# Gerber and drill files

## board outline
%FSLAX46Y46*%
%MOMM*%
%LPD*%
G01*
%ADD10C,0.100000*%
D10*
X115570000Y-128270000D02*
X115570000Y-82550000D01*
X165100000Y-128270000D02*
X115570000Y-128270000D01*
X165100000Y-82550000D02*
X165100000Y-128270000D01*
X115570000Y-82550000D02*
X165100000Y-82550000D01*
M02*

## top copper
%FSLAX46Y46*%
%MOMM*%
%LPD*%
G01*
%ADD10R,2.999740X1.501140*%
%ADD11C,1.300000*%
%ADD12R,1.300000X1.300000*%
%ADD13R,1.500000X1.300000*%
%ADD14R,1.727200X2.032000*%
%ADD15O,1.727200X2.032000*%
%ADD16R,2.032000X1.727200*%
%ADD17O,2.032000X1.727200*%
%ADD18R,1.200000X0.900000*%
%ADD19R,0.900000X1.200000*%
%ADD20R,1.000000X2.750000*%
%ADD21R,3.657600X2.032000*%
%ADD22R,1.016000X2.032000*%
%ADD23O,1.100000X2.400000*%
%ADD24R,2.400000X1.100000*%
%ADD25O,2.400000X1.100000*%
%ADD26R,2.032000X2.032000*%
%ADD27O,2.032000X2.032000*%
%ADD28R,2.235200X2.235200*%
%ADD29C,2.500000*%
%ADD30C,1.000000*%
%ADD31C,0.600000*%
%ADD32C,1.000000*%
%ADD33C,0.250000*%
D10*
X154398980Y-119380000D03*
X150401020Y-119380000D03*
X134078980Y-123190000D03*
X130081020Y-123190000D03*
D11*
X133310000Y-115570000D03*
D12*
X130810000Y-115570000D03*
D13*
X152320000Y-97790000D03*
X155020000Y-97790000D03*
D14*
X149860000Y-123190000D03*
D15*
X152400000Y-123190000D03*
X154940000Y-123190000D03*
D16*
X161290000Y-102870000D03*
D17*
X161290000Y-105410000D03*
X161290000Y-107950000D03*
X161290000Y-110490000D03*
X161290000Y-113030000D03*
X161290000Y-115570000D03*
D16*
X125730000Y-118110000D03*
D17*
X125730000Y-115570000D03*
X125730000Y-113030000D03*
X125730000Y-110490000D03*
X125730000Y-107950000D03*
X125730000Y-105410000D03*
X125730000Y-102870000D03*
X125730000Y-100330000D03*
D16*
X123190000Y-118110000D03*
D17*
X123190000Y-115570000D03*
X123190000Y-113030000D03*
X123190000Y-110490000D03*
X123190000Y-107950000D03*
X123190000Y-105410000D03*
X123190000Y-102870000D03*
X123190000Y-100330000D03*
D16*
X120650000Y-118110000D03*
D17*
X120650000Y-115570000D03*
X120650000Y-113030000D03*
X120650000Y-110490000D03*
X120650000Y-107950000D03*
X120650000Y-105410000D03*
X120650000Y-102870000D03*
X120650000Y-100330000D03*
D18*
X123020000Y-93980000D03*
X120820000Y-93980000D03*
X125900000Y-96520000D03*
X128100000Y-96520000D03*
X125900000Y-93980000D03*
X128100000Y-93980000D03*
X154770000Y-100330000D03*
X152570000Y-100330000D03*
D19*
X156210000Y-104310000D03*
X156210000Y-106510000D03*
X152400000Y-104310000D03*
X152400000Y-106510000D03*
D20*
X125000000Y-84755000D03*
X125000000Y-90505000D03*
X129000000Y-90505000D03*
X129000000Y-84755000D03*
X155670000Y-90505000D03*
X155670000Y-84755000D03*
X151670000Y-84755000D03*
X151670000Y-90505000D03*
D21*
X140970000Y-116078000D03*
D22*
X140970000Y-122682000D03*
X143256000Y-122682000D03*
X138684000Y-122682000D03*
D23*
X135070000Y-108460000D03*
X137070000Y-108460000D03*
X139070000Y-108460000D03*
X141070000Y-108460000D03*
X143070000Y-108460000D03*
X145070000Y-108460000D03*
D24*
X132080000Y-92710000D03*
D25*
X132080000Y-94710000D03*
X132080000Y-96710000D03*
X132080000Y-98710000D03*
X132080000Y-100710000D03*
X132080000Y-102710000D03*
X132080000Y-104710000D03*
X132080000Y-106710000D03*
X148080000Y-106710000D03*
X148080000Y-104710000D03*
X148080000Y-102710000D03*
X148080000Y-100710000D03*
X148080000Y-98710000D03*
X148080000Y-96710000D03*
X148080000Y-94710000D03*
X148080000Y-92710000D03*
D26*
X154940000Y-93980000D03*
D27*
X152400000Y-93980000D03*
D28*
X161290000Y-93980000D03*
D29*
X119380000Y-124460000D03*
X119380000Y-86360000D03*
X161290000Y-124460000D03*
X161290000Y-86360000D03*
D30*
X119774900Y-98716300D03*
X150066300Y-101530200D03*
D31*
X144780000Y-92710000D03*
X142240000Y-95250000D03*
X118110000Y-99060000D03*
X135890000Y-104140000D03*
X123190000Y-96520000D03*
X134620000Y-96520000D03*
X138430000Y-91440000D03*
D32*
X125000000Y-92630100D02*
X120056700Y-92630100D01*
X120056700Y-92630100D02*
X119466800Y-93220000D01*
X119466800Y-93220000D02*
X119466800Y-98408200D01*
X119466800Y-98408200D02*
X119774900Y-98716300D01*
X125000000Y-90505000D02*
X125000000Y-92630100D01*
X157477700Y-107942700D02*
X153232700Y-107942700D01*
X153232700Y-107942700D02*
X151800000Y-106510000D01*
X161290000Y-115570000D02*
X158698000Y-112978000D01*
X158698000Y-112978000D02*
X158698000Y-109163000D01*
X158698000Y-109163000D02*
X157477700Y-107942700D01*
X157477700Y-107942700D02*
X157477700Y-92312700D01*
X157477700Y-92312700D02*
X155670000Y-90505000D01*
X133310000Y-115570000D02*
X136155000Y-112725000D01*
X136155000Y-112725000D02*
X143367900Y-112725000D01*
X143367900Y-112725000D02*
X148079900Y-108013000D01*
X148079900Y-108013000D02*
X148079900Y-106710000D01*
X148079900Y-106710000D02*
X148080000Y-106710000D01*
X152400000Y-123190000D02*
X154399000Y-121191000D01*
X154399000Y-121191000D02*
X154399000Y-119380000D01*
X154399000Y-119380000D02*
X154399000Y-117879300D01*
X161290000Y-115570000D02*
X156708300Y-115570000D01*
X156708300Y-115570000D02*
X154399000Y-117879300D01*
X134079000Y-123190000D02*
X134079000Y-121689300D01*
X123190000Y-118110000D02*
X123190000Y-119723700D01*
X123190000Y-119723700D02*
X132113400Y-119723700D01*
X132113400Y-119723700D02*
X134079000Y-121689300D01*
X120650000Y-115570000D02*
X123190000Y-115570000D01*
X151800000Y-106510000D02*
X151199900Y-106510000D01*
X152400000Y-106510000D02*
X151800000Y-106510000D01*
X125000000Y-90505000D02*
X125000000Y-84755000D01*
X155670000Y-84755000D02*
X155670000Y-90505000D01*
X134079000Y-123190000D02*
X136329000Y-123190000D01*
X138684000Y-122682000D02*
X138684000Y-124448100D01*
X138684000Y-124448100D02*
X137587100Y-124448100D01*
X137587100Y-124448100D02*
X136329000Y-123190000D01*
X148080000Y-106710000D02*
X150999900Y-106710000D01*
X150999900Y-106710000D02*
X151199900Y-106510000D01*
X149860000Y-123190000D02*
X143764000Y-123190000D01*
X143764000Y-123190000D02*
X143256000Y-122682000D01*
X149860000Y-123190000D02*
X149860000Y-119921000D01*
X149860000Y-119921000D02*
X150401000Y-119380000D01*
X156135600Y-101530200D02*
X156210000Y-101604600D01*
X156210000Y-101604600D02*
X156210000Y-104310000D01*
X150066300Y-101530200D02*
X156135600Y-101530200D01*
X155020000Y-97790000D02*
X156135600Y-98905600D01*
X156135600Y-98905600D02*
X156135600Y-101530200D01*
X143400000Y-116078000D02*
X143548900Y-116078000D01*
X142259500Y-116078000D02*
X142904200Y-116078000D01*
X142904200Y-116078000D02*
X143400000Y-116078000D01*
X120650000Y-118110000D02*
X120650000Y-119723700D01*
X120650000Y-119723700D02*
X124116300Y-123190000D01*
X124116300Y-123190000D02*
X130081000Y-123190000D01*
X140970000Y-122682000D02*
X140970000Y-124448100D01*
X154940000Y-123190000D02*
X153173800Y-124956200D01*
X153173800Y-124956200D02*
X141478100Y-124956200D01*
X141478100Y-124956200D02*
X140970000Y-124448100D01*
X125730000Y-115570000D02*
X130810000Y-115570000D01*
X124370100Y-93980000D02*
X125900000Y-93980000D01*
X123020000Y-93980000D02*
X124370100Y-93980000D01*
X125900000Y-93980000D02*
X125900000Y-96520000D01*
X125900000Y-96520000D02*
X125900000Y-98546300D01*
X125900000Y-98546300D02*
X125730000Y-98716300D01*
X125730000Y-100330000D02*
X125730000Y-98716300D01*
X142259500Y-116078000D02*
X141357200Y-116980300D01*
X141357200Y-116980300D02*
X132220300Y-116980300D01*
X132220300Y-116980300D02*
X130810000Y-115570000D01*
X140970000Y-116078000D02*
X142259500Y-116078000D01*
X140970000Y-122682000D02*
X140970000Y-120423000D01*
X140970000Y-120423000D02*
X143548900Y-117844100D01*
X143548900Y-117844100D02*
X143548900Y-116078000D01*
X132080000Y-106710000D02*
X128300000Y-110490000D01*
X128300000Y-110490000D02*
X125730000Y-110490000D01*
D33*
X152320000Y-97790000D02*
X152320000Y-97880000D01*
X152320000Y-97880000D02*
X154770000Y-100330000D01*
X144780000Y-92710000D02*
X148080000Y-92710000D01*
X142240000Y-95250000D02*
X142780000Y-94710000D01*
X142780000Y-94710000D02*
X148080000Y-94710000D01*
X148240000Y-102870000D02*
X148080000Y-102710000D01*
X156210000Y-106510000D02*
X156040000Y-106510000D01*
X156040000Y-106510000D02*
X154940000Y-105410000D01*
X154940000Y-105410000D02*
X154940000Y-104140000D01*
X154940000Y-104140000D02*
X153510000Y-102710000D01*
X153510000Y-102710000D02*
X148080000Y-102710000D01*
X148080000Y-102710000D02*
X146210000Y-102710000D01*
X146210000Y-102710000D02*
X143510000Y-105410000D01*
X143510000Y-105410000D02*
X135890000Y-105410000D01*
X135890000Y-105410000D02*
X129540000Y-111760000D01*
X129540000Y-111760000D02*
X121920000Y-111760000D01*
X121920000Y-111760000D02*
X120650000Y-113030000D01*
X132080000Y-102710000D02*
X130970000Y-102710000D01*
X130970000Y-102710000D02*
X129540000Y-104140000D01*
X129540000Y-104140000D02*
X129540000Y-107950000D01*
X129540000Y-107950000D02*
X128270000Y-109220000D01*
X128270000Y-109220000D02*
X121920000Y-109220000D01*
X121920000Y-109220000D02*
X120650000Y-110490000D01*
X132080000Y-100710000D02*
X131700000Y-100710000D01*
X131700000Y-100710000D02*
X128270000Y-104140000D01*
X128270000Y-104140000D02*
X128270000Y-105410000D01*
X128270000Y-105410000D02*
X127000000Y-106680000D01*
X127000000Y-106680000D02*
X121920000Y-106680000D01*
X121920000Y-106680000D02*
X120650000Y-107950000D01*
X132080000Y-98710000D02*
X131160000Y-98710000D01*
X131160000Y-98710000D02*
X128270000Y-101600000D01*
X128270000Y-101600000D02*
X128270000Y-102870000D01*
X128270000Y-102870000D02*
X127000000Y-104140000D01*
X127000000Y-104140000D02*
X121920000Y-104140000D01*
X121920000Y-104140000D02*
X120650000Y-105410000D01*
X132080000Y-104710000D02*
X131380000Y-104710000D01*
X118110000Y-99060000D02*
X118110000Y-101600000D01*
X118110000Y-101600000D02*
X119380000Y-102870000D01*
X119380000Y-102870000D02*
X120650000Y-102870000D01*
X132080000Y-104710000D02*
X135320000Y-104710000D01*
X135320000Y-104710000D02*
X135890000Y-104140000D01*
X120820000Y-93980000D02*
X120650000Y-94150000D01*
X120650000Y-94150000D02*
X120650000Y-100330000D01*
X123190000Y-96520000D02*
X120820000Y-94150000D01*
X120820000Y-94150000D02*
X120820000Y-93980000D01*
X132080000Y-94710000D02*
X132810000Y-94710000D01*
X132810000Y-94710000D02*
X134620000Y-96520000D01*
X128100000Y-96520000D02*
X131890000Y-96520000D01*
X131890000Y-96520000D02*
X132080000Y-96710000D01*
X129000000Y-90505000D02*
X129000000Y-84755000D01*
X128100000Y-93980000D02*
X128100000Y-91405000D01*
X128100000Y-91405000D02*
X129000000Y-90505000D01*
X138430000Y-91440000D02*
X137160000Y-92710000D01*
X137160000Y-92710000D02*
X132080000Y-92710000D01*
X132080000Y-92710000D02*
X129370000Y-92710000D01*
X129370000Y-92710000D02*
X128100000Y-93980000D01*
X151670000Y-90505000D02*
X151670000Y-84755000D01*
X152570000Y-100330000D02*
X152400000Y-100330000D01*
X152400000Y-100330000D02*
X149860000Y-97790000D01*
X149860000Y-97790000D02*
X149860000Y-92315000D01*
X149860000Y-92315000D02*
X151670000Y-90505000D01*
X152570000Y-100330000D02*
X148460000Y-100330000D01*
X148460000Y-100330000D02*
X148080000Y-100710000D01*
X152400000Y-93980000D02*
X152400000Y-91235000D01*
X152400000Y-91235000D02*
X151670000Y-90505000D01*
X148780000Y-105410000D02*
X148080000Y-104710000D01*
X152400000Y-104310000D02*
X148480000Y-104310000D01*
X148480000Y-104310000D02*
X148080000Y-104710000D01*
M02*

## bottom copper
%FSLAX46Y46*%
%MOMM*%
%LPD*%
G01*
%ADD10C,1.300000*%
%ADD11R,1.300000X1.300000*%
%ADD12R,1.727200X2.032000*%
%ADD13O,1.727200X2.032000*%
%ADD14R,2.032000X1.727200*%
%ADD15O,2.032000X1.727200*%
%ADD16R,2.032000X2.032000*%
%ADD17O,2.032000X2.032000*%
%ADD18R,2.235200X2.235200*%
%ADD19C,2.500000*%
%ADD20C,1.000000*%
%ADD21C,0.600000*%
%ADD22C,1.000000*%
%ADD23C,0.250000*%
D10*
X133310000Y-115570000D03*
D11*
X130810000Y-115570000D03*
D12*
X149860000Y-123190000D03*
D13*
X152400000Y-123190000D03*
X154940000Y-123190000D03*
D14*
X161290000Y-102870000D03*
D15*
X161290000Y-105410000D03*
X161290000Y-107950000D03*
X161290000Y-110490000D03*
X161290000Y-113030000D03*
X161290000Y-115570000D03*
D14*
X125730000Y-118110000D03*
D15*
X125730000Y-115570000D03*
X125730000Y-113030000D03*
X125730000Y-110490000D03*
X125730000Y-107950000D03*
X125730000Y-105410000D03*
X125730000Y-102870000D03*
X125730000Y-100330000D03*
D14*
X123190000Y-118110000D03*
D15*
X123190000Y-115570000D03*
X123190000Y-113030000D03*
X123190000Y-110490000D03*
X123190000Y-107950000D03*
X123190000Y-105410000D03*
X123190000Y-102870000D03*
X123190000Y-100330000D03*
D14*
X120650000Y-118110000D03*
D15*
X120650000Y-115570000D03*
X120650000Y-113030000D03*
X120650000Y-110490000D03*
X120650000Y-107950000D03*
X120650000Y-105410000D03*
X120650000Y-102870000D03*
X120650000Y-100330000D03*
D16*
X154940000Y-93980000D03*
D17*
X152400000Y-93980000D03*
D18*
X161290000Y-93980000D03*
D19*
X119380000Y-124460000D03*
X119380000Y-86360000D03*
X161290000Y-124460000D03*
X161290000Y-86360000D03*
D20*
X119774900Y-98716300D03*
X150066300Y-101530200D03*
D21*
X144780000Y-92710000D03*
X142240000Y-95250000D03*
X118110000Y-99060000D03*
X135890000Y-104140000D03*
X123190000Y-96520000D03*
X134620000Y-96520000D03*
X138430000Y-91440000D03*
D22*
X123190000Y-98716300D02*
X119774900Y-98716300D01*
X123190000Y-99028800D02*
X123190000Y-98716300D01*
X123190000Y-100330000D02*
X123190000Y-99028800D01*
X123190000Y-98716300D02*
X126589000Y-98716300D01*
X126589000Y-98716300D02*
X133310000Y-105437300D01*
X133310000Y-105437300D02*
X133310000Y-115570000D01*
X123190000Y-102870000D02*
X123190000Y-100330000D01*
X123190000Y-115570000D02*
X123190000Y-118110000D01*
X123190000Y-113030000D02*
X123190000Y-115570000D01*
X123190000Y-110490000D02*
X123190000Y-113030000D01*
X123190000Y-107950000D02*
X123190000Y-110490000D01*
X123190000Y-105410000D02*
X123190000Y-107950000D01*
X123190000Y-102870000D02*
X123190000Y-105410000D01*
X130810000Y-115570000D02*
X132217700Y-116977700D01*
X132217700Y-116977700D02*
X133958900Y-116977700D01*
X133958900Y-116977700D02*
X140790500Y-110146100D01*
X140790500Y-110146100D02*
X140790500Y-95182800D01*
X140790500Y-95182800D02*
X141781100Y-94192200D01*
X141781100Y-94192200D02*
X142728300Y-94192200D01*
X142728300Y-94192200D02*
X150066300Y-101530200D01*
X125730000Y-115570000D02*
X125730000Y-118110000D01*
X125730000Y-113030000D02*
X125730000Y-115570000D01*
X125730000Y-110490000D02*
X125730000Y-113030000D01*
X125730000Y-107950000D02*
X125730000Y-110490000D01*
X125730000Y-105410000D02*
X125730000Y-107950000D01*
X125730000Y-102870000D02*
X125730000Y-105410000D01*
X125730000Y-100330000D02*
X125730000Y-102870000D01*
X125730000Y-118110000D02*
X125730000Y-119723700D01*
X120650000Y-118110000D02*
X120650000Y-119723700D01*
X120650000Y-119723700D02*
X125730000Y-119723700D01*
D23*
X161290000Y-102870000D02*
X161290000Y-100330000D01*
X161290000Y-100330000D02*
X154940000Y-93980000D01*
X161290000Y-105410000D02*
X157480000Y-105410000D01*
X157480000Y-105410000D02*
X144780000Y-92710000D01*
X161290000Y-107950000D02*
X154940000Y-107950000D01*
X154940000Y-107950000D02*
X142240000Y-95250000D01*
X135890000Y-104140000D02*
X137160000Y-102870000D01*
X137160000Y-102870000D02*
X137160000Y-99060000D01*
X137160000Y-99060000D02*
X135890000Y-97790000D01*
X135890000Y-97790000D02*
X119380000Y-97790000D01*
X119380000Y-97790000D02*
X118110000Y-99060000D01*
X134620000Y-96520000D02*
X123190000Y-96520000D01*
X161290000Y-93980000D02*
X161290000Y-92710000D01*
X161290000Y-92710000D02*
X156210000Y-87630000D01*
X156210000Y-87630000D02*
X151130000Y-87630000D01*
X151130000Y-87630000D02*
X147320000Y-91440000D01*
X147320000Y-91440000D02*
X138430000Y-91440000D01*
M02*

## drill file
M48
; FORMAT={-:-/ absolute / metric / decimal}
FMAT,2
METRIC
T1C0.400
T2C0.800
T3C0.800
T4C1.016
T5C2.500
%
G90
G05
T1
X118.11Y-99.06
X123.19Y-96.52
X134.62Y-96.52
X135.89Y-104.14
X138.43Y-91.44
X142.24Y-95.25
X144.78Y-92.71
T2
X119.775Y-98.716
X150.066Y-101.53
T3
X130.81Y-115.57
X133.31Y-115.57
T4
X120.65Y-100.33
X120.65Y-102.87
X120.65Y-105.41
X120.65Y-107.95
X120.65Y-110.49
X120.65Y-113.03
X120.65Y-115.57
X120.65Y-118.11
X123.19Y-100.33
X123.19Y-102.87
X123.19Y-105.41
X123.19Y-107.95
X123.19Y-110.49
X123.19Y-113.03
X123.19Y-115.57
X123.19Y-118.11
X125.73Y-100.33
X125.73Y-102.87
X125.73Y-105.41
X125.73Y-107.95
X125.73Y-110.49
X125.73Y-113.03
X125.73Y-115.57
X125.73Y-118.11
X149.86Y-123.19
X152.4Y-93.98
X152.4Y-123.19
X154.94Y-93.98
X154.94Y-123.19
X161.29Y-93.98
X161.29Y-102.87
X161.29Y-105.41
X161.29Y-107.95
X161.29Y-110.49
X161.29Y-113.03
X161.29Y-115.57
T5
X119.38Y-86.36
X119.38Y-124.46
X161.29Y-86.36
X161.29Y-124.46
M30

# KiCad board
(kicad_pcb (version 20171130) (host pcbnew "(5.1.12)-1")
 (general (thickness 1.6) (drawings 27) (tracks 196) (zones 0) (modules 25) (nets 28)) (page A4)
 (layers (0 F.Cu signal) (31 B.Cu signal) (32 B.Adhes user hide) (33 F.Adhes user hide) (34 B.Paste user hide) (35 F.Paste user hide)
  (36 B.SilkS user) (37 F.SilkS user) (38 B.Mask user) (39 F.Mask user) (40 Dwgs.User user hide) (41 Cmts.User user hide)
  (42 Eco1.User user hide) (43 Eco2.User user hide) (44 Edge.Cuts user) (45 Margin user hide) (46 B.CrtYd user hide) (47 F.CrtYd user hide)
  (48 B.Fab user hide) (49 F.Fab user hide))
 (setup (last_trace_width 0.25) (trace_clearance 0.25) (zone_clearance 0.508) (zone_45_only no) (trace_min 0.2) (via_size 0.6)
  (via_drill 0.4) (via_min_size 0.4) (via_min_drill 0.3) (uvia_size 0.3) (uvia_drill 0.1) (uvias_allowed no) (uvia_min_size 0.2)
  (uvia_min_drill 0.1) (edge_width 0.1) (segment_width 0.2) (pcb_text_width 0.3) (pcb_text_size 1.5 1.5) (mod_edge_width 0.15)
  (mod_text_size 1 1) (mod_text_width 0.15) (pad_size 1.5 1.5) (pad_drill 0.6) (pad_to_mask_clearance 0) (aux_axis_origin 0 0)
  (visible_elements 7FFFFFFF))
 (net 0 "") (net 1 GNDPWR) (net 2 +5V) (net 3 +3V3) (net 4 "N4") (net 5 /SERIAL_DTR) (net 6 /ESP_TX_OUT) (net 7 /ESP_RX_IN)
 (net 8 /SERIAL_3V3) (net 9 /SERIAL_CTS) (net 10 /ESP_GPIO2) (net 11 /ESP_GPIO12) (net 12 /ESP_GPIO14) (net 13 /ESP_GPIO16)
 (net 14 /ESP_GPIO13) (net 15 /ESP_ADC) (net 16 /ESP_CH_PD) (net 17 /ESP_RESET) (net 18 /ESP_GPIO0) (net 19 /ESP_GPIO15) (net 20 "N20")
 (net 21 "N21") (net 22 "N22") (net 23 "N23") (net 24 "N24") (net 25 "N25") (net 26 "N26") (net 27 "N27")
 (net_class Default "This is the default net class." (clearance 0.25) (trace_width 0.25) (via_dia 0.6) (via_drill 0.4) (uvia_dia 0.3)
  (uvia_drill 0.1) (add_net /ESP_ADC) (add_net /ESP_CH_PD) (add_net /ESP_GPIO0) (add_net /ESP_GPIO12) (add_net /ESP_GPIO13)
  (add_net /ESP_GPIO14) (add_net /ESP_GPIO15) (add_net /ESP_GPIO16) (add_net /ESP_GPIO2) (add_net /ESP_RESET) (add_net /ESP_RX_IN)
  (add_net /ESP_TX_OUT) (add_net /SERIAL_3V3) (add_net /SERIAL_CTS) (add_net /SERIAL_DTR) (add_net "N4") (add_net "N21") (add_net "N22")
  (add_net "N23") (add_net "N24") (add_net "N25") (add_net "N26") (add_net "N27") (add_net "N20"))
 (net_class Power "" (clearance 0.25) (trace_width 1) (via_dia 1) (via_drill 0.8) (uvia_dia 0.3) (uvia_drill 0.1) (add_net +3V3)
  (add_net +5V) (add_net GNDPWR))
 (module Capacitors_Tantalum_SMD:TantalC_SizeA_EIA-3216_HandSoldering (layer F.Cu) (at 152.4 119.38)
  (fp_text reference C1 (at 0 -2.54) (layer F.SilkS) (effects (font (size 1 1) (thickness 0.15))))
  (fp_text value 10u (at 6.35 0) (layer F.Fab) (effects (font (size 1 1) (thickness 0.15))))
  (pad 2 smd rect (at 1.99898 0) (size 2.99974 1.50114) (layers F.Cu F.Paste F.Mask) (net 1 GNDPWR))
  (pad 1 smd rect (at -1.99898 0) (size 2.99974 1.50114) (layers F.Cu F.Paste F.Mask) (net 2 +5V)))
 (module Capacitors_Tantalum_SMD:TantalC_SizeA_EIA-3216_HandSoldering (layer F.Cu) (at 132.08 123.19)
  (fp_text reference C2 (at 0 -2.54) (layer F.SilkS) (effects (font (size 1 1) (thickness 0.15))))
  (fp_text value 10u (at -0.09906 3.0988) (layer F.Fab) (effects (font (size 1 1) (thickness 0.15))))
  (pad 2 smd rect (at 1.99898 0) (size 2.99974 1.50114) (layers F.Cu F.Paste F.Mask) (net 1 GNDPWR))
  (pad 1 smd rect (at -1.99898 0) (size 2.99974 1.50114) (layers F.Cu F.Paste F.Mask) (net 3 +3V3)))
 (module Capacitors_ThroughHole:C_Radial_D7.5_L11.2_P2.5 (layer F.Cu) (at 130.81 115.57)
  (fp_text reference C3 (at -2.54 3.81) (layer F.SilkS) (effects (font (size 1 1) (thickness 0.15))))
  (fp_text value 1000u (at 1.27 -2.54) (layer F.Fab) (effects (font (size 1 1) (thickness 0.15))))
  (pad 2 thru_hole circle (at 2.5 0) (size 1.3 1.3) (drill 0.8) (layers *.Cu *.Mask F.SilkS) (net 1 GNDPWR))
  (pad 1 thru_hole rect (at 0 0) (size 1.3 1.3) (drill 0.8) (layers *.Cu *.Mask F.SilkS) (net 3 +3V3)))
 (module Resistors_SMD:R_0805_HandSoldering (layer F.Cu) (at 153.67 97.79)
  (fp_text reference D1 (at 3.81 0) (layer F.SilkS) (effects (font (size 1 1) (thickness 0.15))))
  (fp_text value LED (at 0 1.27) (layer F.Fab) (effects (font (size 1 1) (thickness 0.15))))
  (pad 1 smd rect (at -1.35 0) (size 1.5 1.3) (layers F.Cu F.Paste F.Mask) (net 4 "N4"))
  (pad 2 smd rect (at 1.35 0) (size 1.5 1.3) (layers F.Cu F.Paste F.Mask) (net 3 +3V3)))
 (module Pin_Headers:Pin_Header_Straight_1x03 (layer F.Cu) (at 149.86 123.19 90)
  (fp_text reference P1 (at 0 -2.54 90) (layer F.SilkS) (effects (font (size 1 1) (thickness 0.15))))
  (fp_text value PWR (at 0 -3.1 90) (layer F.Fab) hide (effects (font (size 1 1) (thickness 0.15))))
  (pad 1 thru_hole rect (at 0 0 90) (size 2.032 1.7272) (drill 1.016) (layers *.Cu *.Mask F.SilkS) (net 2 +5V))
  (pad 2 thru_hole oval (at 0 2.54 90) (size 2.032 1.7272) (drill 1.016) (layers *.Cu *.Mask F.SilkS) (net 1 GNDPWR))
  (pad 3 thru_hole oval (at 0 5.08 90) (size 2.032 1.7272) (drill 1.016) (layers *.Cu *.Mask F.SilkS) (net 3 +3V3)))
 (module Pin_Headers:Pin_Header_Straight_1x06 (layer F.Cu) (at 161.29 102.87)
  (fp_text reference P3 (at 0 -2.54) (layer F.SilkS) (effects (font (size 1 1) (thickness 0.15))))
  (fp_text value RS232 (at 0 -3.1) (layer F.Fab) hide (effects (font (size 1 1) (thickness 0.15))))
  (pad 1 thru_hole rect (at 0 0) (size 2.032 1.7272) (drill 1.016) (layers *.Cu *.Mask F.SilkS) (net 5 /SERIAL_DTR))
  (pad 2 thru_hole oval (at 0 2.54) (size 2.032 1.7272) (drill 1.016) (layers *.Cu *.Mask F.SilkS) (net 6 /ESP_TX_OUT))
  (pad 3 thru_hole oval (at 0 5.08) (size 2.032 1.7272) (drill 1.016) (layers *.Cu *.Mask F.SilkS) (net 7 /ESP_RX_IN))
  (pad 4 thru_hole oval (at 0 7.62) (size 2.032 1.7272) (drill 1.016) (layers *.Cu *.Mask F.SilkS) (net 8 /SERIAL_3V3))
  (pad 5 thru_hole oval (at 0 10.16) (size 2.032 1.7272) (drill 1.016) (layers *.Cu *.Mask F.SilkS) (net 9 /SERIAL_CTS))
  (pad 6 thru_hole oval (at 0 12.7) (size 2.032 1.7272) (drill 1.016) (layers *.Cu *.Mask F.SilkS) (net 1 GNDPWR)))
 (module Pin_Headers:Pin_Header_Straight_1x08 (layer F.Cu) (at 125.73 118.11 180)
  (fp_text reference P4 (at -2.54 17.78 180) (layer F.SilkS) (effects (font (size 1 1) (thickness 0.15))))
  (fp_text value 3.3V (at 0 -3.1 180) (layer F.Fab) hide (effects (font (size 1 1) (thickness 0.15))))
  (pad 1 thru_hole rect (at 0 0 180) (size 2.032 1.7272) (drill 1.016) (layers *.Cu *.Mask F.SilkS) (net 3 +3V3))
  (pad 2 thru_hole oval (at 0 2.54 180) (size 2.032 1.7272) (drill 1.016) (layers *.Cu *.Mask F.SilkS) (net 3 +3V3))
  (pad 3 thru_hole oval (at 0 5.08 180) (size 2.032 1.7272) (drill 1.016) (layers *.Cu *.Mask F.SilkS) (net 3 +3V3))
  (pad 4 thru_hole oval (at 0 7.62 180) (size 2.032 1.7272) (drill 1.016) (layers *.Cu *.Mask F.SilkS) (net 3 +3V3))
  (pad 5 thru_hole oval (at 0 10.16 180) (size 2.032 1.7272) (drill 1.016) (layers *.Cu *.Mask F.SilkS) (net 3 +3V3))
  (pad 6 thru_hole oval (at 0 12.7 180) (size 2.032 1.7272) (drill 1.016) (layers *.Cu *.Mask F.SilkS) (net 3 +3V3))
  (pad 7 thru_hole oval (at 0 15.24 180) (size 2.032 1.7272) (drill 1.016) (layers *.Cu *.Mask F.SilkS) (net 3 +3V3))
  (pad 8 thru_hole oval (at 0 17.78 180) (size 2.032 1.7272) (drill 1.016) (layers *.Cu *.Mask F.SilkS) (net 3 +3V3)))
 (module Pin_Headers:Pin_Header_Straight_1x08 (layer F.Cu) (at 123.19 118.11 180)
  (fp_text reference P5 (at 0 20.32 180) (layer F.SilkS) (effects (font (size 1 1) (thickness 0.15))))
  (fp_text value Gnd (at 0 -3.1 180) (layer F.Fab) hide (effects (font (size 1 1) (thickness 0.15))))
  (pad 1 thru_hole rect (at 0 0 180) (size 2.032 1.7272) (drill 1.016) (layers *.Cu *.Mask F.SilkS) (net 1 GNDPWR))
  (pad 2 thru_hole oval (at 0 2.54 180) (size 2.032 1.7272) (drill 1.016) (layers *.Cu *.Mask F.SilkS) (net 1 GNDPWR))
  (pad 3 thru_hole oval (at 0 5.08 180) (size 2.032 1.7272) (drill 1.016) (layers *.Cu *.Mask F.SilkS) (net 1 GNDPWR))
  (pad 4 thru_hole oval (at 0 7.62 180) (size 2.032 1.7272) (drill 1.016) (layers *.Cu *.Mask F.SilkS) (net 1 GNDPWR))
  (pad 5 thru_hole oval (at 0 10.16 180) (size 2.032 1.7272) (drill 1.016) (layers *.Cu *.Mask F.SilkS) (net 1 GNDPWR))
  (pad 6 thru_hole oval (at 0 12.7 180) (size 2.032 1.7272) (drill 1.016) (layers *.Cu *.Mask F.SilkS) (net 1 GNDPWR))
  (pad 7 thru_hole oval (at 0 15.24 180) (size 2.032 1.7272) (drill 1.016) (layers *.Cu *.Mask F.SilkS) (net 1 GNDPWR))
  (pad 8 thru_hole oval (at 0 17.78 180) (size 2.032 1.7272) (drill 1.016) (layers *.Cu *.Mask F.SilkS) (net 1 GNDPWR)))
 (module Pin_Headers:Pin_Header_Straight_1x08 (layer F.Cu) (at 120.65 118.11 180)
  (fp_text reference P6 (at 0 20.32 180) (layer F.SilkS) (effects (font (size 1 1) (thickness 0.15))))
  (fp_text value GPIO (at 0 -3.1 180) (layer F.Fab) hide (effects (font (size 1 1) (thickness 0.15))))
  (pad 1 thru_hole rect (at 0 0 180) (size 2.032 1.7272) (drill 1.016) (layers *.Cu *.Mask F.SilkS) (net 3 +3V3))
  (pad 2 thru_hole oval (at 0 2.54 180) (size 2.032 1.7272) (drill 1.016) (layers *.Cu *.Mask F.SilkS) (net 1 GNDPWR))
  (pad 3 thru_hole oval (at 0 5.08 180) (size 2.032 1.7272) (drill 1.016) (layers *.Cu *.Mask F.SilkS) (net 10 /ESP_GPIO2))
  (pad 4 thru_hole oval (at 0 7.62 180) (size 2.032 1.7272) (drill 1.016) (layers *.Cu *.Mask F.SilkS) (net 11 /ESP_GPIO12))
  (pad 5 thru_hole oval (at 0 10.16 180) (size 2.032 1.7272) (drill 1.016) (layers *.Cu *.Mask F.SilkS) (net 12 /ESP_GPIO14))
  (pad 6 thru_hole oval (at 0 12.7 180) (size 2.032 1.7272) (drill 1.016) (layers *.Cu *.Mask F.SilkS) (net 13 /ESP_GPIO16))
  (pad 7 thru_hole oval (at 0 15.24 180) (size 2.032 1.7272) (drill 1.016) (layers *.Cu *.Mask F.SilkS) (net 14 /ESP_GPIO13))
  (pad 8 thru_hole oval (at 0 17.78 180) (size 2.032 1.7272) (drill 1.016) (layers *.Cu *.Mask F.SilkS) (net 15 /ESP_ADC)))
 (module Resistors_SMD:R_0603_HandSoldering (layer F.Cu) (at 121.92 93.98 180)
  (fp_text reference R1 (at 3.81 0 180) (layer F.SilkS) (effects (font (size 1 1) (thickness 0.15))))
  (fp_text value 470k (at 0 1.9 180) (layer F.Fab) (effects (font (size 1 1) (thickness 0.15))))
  (pad 1 smd rect (at -1.1 0 180) (size 1.2 0.9) (layers F.Cu F.Paste F.Mask) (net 3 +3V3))
  (pad 2 smd rect (at 1.1 0 180) (size 1.2 0.9) (layers F.Cu F.Paste F.Mask) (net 15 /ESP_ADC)))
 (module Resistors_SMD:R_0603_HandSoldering (layer F.Cu) (at 127 96.52)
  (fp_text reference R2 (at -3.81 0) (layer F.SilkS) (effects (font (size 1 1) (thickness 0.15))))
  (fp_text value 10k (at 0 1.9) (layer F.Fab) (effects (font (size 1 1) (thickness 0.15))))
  (pad 1 smd rect (at -1.1 0) (size 1.2 0.9) (layers F.Cu F.Paste F.Mask) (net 3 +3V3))
  (pad 2 smd rect (at 1.1 0) (size 1.2 0.9) (layers F.Cu F.Paste F.Mask) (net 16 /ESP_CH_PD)))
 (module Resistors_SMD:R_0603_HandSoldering (layer F.Cu) (at 127 93.98)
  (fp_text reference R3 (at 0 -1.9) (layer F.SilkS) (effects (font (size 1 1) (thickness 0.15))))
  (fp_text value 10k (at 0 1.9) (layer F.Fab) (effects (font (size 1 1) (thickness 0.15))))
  (pad 1 smd rect (at -1.1 0) (size 1.2 0.9) (layers F.Cu F.Paste F.Mask) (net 3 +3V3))
  (pad 2 smd rect (at 1.1 0) (size 1.2 0.9) (layers F.Cu F.Paste F.Mask) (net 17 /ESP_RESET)))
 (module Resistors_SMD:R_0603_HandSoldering (layer F.Cu) (at 153.67 100.33 180)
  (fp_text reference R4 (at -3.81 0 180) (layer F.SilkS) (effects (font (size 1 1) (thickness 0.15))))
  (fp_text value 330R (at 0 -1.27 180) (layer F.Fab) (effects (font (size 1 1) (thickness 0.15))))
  (pad 1 smd rect (at -1.1 0 180) (size 1.2 0.9) (layers F.Cu F.Paste F.Mask) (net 4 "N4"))
  (pad 2 smd rect (at 1.1 0 180) (size 1.2 0.9) (layers F.Cu F.Paste F.Mask) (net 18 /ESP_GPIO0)))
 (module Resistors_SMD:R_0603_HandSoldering (layer F.Cu) (at 156.21 105.41 270)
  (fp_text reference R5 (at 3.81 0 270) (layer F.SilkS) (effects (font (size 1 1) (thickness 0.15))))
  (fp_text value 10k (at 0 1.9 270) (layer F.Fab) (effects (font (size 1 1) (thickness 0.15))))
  (pad 1 smd rect (at -1.1 0 270) (size 1.2 0.9) (layers F.Cu F.Paste F.Mask) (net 3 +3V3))
  (pad 2 smd rect (at 1.1 0 270) (size 1.2 0.9) (layers F.Cu F.Paste F.Mask) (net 10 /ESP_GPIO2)))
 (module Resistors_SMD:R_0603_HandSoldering (layer F.Cu) (at 152.4 105.41 270)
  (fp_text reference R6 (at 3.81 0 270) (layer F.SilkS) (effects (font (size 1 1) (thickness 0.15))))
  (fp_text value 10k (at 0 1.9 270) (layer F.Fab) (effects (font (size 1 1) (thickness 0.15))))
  (pad 1 smd rect (at -1.1 0 270) (size 1.2 0.9) (layers F.Cu F.Paste F.Mask) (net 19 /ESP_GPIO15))
  (pad 2 smd rect (at 1.1 0 270) (size 1.2 0.9) (layers F.Cu F.Paste F.Mask) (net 1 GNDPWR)))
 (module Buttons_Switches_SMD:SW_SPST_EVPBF (layer F.Cu) (at 127 87.63 90)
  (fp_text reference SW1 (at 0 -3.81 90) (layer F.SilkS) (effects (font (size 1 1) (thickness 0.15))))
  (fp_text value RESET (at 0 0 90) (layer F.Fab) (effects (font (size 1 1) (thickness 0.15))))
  (pad 1 smd rect (at 2.875 -2 90) (size 2.75 1) (layers F.Cu F.Paste F.Mask) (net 1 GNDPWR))
  (pad 1 smd rect (at -2.875 -2 90) (size 2.75 1) (layers F.Cu F.Paste F.Mask) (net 1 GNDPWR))
  (pad 2 smd rect (at -2.875 2 90) (size 2.75 1) (layers F.Cu F.Paste F.Mask) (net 17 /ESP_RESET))
  (pad 2 smd rect (at 2.875 2 90) (size 2.75 1) (layers F.Cu F.Paste F.Mask) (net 17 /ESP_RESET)))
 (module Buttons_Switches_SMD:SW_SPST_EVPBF (layer F.Cu) (at 153.67 87.63 270)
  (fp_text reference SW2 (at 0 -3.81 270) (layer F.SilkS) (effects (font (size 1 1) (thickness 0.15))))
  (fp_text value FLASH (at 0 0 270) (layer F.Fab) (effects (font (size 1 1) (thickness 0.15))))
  (pad 1 smd rect (at 2.875 -2 270) (size 2.75 1) (layers F.Cu F.Paste F.Mask) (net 1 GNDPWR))
  (pad 1 smd rect (at -2.875 -2 270) (size 2.75 1) (layers F.Cu F.Paste F.Mask) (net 1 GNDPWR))
  (pad 2 smd rect (at -2.875 2 270) (size 2.75 1) (layers F.Cu F.Paste F.Mask) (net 18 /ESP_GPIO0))
  (pad 2 smd rect (at 2.875 2 270) (size 2.75 1) (layers F.Cu F.Paste F.Mask) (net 18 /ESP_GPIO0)))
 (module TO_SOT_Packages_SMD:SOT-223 (layer F.Cu) (at 140.97 119.38)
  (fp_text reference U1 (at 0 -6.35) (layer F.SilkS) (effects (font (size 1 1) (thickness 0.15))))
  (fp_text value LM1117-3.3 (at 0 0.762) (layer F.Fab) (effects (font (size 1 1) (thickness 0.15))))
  (pad 4 smd rect (at 0 -3.302) (size 3.6576 2.032) (layers F.Cu F.Paste F.Mask) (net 3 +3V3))
  (pad 2 smd rect (at 0 3.302) (size 1.016 2.032) (layers F.Cu F.Paste F.Mask) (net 3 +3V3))
  (pad 3 smd rect (at 2.286 3.302) (size 1.016 2.032) (layers F.Cu F.Paste F.Mask) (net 2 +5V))
  (pad 1 smd rect (at -2.286 3.302) (size 1.016 2.032) (layers F.Cu F.Paste F.Mask) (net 1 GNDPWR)))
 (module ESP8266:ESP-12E (layer F.Cu) (at 132.08 92.71)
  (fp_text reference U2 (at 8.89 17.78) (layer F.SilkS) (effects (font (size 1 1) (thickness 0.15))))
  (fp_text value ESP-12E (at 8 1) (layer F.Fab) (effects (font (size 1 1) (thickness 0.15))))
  (pad 9 smd oval (at 2.99 15.75 90) (size 2.4 1.1) (layers F.Cu F.Paste F.Mask) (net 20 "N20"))
  (pad 10 smd oval (at 4.99 15.75 90) (size 2.4 1.1) (layers F.Cu F.Paste F.Mask) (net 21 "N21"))
  (pad 11 smd oval (at 6.99 15.75 90) (size 2.4 1.1) (layers F.Cu F.Paste F.Mask) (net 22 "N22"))
  (pad 12 smd oval (at 8.99 15.75 90) (size 2.4 1.1) (layers F.Cu F.Paste F.Mask) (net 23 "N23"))
  (pad 13 smd oval (at 10.99 15.75 90) (size 2.4 1.1) (layers F.Cu F.Paste F.Mask) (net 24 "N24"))
  (pad 14 smd oval (at 12.99 15.75 90) (size 2.4 1.1) (layers F.Cu F.Paste F.Mask) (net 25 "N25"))
  (pad 1 smd rect (at 0 0) (size 2.4 1.1) (layers F.Cu F.Paste F.Mask) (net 17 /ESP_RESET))
  (pad 2 smd oval (at 0 2) (size 2.4 1.1) (layers F.Cu F.Paste F.Mask) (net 15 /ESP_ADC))
  (pad 3 smd oval (at 0 4) (size 2.4 1.1) (layers F.Cu F.Paste F.Mask) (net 16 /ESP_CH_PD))
  (pad 4 smd oval (at 0 6) (size 2.4 1.1) (layers F.Cu F.Paste F.Mask) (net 13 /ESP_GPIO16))
  (pad 5 smd oval (at 0 8) (size 2.4 1.1) (layers F.Cu F.Paste F.Mask) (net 12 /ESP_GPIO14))
  (pad 6 smd oval (at 0 10) (size 2.4 1.1) (layers F.Cu F.Paste F.Mask) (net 11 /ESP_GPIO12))
  (pad 7 smd oval (at 0 12) (size 2.4 1.1) (layers F.Cu F.Paste F.Mask) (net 14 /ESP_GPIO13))
  (pad 8 smd oval (at 0 14) (size 2.4 1.1) (layers F.Cu F.Paste F.Mask) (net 3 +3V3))
  (pad 15 smd oval (at 16 14) (size 2.4 1.1) (layers F.Cu F.Paste F.Mask) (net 1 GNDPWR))
  (pad 16 smd oval (at 16 12) (size 2.4 1.1) (layers F.Cu F.Paste F.Mask) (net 19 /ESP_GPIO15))
  (pad 17 smd oval (at 16 10) (size 2.4 1.1) (layers F.Cu F.Paste F.Mask) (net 10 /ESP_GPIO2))
  (pad 18 smd oval (at 16 8) (size 2.4 1.1) (layers F.Cu F.Paste F.Mask) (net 18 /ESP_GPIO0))
  (pad 19 smd oval (at 16 6) (size 2.4 1.1) (layers F.Cu F.Paste F.Mask) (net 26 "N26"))
  (pad 20 smd oval (at 16 4) (size 2.4 1.1) (layers F.Cu F.Paste F.Mask) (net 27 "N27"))
  (pad 21 smd oval (at 16 2) (size 2.4 1.1) (layers F.Cu F.Paste F.Mask) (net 7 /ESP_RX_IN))
  (pad 22 smd oval (at 16 0) (size 2.4 1.1) (layers F.Cu F.Paste F.Mask) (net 6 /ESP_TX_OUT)))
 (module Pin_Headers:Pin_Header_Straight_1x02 (layer F.Cu) (at 154.94 93.98 270)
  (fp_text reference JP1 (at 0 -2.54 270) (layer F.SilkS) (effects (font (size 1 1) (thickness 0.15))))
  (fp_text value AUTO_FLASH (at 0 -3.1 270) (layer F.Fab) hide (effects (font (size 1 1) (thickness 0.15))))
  (pad 1 thru_hole rect (at 0 0 270) (size 2.032 2.032) (drill 1.016) (layers *.Cu *.Mask F.SilkS) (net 5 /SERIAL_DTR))
  (pad 2 thru_hole oval (at 0 2.54 270) (size 2.032 2.032) (drill 1.016) (layers *.Cu *.Mask F.SilkS) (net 18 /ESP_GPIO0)))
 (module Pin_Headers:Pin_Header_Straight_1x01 (layer F.Cu) (at 161.29 93.98)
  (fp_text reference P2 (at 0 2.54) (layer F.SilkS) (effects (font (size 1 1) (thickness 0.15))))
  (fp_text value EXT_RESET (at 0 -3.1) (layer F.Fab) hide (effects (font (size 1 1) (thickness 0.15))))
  (pad 1 thru_hole rect (at 0 0) (size 2.2352 2.2352) (drill 1.016) (layers *.Cu *.Mask F.SilkS) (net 17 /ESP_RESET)))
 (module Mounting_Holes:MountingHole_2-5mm (layer F.Cu) (at 119.38 124.46)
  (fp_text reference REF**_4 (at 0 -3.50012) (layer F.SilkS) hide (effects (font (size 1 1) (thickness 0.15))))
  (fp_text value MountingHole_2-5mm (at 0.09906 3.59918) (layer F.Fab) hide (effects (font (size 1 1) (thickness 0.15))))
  (pad 1 thru_hole circle (at 0 0) (size 2.5 2.5) (drill 2.5) (layers *.Cu *.Mask)))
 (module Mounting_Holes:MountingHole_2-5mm (layer F.Cu) (at 119.38 86.36)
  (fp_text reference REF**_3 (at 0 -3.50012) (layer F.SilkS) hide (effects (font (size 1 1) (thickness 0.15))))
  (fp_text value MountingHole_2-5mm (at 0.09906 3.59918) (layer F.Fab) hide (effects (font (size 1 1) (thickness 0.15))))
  (pad 1 thru_hole circle (at 0 0) (size 2.5 2.5) (drill 2.5) (layers *.Cu *.Mask)))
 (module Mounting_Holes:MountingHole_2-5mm (layer F.Cu) (at 161.29 124.46)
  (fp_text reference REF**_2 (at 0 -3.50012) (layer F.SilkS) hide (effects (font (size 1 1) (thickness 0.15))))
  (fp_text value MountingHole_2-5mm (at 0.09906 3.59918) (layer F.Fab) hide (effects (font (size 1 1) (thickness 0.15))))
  (pad 1 thru_hole circle (at 0 0) (size 2.5 2.5) (drill 2.5) (layers *.Cu *.Mask)))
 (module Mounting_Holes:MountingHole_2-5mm (layer F.Cu) (at 161.29 86.36)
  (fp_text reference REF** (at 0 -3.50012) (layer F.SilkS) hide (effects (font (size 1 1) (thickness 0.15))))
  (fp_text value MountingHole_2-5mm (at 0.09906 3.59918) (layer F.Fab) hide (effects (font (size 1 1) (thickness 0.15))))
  (pad 1 thru_hole circle (at 0 0) (size 2.5 2.5) (drill 2.5) (layers *.Cu *.Mask)))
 (gr_line (start 115.57 128.27) (end 115.57 82.55) (angle 90) (layer Edge.Cuts) (width 0.1))
 (gr_line (start 165.1 128.27) (end 115.57 128.27) (angle 90) (layer Edge.Cuts) (width 0.1))
 (gr_line (start 165.1 82.55) (end 165.1 128.27) (angle 90) (layer Edge.Cuts) (width 0.1))
 (gr_line (start 115.57 82.55) (end 165.1 82.55) (angle 90) (layer Edge.Cuts) (width 0.1))
 (segment (start 125 92.6301) (end 120.0567 92.6301) (width 1) (layer F.Cu) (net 1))
 (segment (start 120.0567 92.6301) (end 119.4668 93.22) (width 1) (layer F.Cu) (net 1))
 (segment (start 119.4668 93.22) (end 119.4668 98.4082) (width 1) (layer F.Cu) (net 1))
 (segment (start 119.4668 98.4082) (end 119.7749 98.7163) (width 1) (layer F.Cu) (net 1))
 (segment (start 123.19 98.7163) (end 119.7749 98.7163) (width 1) (layer B.Cu) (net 1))
 (segment (start 125 90.505) (end 125 92.6301) (width 1) (layer F.Cu) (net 1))
 (segment (start 123.19 99.0288) (end 123.19 98.7163) (width 1) (layer B.Cu) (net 1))
 (segment (start 123.19 100.33) (end 123.19 99.0288) (width 1) (layer B.Cu) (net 1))
 (segment (start 157.4777 107.9427) (end 153.2327 107.9427) (width 1) (layer F.Cu) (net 1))
 (segment (start 153.2327 107.9427) (end 151.8 106.51) (width 1) (layer F.Cu) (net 1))
 (segment (start 161.29 115.57) (end 158.698 112.978) (width 1) (layer F.Cu) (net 1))
 (segment (start 158.698 112.978) (end 158.698 109.163) (width 1) (layer F.Cu) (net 1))
 (segment (start 158.698 109.163) (end 157.4777 107.9427) (width 1) (layer F.Cu) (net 1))
 (segment (start 157.4777 107.9427) (end 157.4777 92.3127) (width 1) (layer F.Cu) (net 1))
 (segment (start 157.4777 92.3127) (end 155.67 90.505) (width 1) (layer F.Cu) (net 1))
 (segment (start 123.19 98.7163) (end 126.589 98.7163) (width 1) (layer B.Cu) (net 1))
 (segment (start 126.589 98.7163) (end 133.31 105.4373) (width 1) (layer B.Cu) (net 1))
 (segment (start 133.31 105.4373) (end 133.31 115.57) (width 1) (layer B.Cu) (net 1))
 (segment (start 123.19 102.87) (end 123.19 100.33) (width 1) (layer B.Cu) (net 1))
 (segment (start 133.31 115.57) (end 136.155 112.725) (width 1) (layer F.Cu) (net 1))
 (segment (start 136.155 112.725) (end 143.3679 112.725) (width 1) (layer F.Cu) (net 1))
 (segment (start 143.3679 112.725) (end 148.0799 108.013) (width 1) (layer F.Cu) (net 1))
 (segment (start 148.0799 108.013) (end 148.0799 106.71) (width 1) (layer F.Cu) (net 1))
 (segment (start 148.0799 106.71) (end 148.08 106.71) (width 1) (layer F.Cu) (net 1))
 (segment (start 152.4 123.19) (end 154.399 121.191) (width 1) (layer F.Cu) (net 1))
 (segment (start 154.399 121.191) (end 154.399 119.38) (width 1) (layer F.Cu) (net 1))
 (segment (start 154.399 119.38) (end 154.399 117.8793) (width 1) (layer F.Cu) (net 1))
 (segment (start 161.29 115.57) (end 156.7083 115.57) (width 1) (layer F.Cu) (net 1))
 (segment (start 156.7083 115.57) (end 154.399 117.8793) (width 1) (layer F.Cu) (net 1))
 (segment (start 134.079 123.19) (end 134.079 121.6893) (width 1) (layer F.Cu) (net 1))
 (segment (start 123.19 118.11) (end 123.19 119.7237) (width 1) (layer F.Cu) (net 1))
 (segment (start 123.19 119.7237) (end 132.1134 119.7237) (width 1) (layer F.Cu) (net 1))
 (segment (start 132.1134 119.7237) (end 134.079 121.6893) (width 1) (layer F.Cu) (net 1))
 (segment (start 123.19 115.57) (end 123.19 118.11) (width 1) (layer B.Cu) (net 1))
 (segment (start 123.19 113.03) (end 123.19 115.57) (width 1) (layer B.Cu) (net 1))
 (segment (start 123.19 110.49) (end 123.19 113.03) (width 1) (layer B.Cu) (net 1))
 (segment (start 123.19 107.95) (end 123.19 110.49) (width 1) (layer B.Cu) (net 1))
 (segment (start 123.19 105.41) (end 123.19 107.95) (width 1) (layer B.Cu) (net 1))
 (segment (start 123.19 102.87) (end 123.19 105.41) (width 1) (layer B.Cu) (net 1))
 (segment (start 120.65 115.57) (end 123.19 115.57) (width 1) (layer F.Cu) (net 1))
 (segment (start 151.8 106.51) (end 151.1999 106.51) (width 1) (layer F.Cu) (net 1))
 (segment (start 152.4 106.51) (end 151.8 106.51) (width 1) (layer F.Cu) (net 1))
 (segment (start 125 90.505) (end 125 84.755) (width 1) (layer F.Cu) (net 1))
 (segment (start 155.67 84.755) (end 155.67 90.505) (width 1) (layer F.Cu) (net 1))
 (segment (start 134.079 123.19) (end 136.329 123.19) (width 1) (layer F.Cu) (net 1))
 (segment (start 138.684 122.682) (end 138.684 124.4481) (width 1) (layer F.Cu) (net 1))
 (segment (start 138.684 124.4481) (end 137.5871 124.4481) (width 1) (layer F.Cu) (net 1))
 (segment (start 137.5871 124.4481) (end 136.329 123.19) (width 1) (layer F.Cu) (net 1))
 (segment (start 148.08 106.71) (end 150.9999 106.71) (width 1) (layer F.Cu) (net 1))
 (segment (start 150.9999 106.71) (end 151.1999 106.51) (width 1) (layer F.Cu) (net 1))
 (via (at 119.7749 98.7163) (size 1) (drill 0.8) (layers F.Cu B.Cu) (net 1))
 (segment (start 149.86 123.19) (end 143.764 123.19) (width 1) (layer F.Cu) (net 2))
 (segment (start 143.764 123.19) (end 143.256 122.682) (width 1) (layer F.Cu) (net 2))
 (segment (start 149.86 123.19) (end 149.86 119.921) (width 1) (layer F.Cu) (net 2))
 (segment (start 149.86 119.921) (end 150.401 119.38) (width 1) (layer F.Cu) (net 2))
 (segment (start 156.1356 101.5302) (end 156.21 101.6046) (width 1) (layer F.Cu) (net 3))
 (segment (start 156.21 101.6046) (end 156.21 104.31) (width 1) (layer F.Cu) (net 3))
 (segment (start 150.0663 101.5302) (end 156.1356 101.5302) (width 1) (layer F.Cu) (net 3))
 (segment (start 155.02 97.79) (end 156.1356 98.9056) (width 1) (layer F.Cu) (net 3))
 (segment (start 156.1356 98.9056) (end 156.1356 101.5302) (width 1) (layer F.Cu) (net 3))
 (segment (start 130.81 115.57) (end 132.2177 116.9777) (width 1) (layer B.Cu) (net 3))
 (segment (start 132.2177 116.9777) (end 133.9589 116.9777) (width 1) (layer B.Cu) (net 3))
 (segment (start 133.9589 116.9777) (end 140.7905 110.1461) (width 1) (layer B.Cu) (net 3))
 (segment (start 140.7905 110.1461) (end 140.7905 95.1828) (width 1) (layer B.Cu) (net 3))
 (segment (start 140.7905 95.1828) (end 141.7811 94.1922) (width 1) (layer B.Cu) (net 3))
 (segment (start 141.7811 94.1922) (end 142.7283 94.1922) (width 1) (layer B.Cu) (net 3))
 (segment (start 142.7283 94.1922) (end 150.0663 101.5302) (width 1) (layer B.Cu) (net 3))
 (segment (start 143.4 116.078) (end 143.5489 116.078) (width 1) (layer F.Cu) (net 3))
 (segment (start 142.2595 116.078) (end 142.9042 116.078) (width 1) (layer F.Cu) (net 3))
 (segment (start 142.9042 116.078) (end 143.4 116.078) (width 1) (layer F.Cu) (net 3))
 (segment (start 120.65 118.11) (end 120.65 119.7237) (width 1) (layer F.Cu) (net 3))
 (segment (start 120.65 119.7237) (end 124.1163 123.19) (width 1) (layer F.Cu) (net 3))
 (segment (start 124.1163 123.19) (end 130.081 123.19) (width 1) (layer F.Cu) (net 3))
 (segment (start 140.97 122.682) (end 140.97 124.4481) (width 1) (layer F.Cu) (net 3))
 (segment (start 154.94 123.19) (end 153.1738 124.9562) (width 1) (layer F.Cu) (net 3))
 (segment (start 153.1738 124.9562) (end 141.4781 124.9562) (width 1) (layer F.Cu) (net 3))
 (segment (start 141.4781 124.9562) (end 140.97 124.4481) (width 1) (layer F.Cu) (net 3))
 (segment (start 125.73 115.57) (end 130.81 115.57) (width 1) (layer F.Cu) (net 3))
 (segment (start 125.73 115.57) (end 125.73 118.11) (width 1) (layer B.Cu) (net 3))
 (segment (start 125.73 113.03) (end 125.73 115.57) (width 1) (layer B.Cu) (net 3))
 (segment (start 125.73 110.49) (end 125.73 113.03) (width 1) (layer B.Cu) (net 3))
 (segment (start 125.73 107.95) (end 125.73 110.49) (width 1) (layer B.Cu) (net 3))
 (segment (start 125.73 105.41) (end 125.73 107.95) (width 1) (layer B.Cu) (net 3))
 (segment (start 125.73 102.87) (end 125.73 105.41) (width 1) (layer B.Cu) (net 3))
 (segment (start 125.73 100.33) (end 125.73 102.87) (width 1) (layer B.Cu) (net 3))
 (segment (start 125.73 118.11) (end 125.73 119.7237) (width 1) (layer B.Cu) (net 3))
 (segment (start 120.65 118.11) (end 120.65 119.7237) (width 1) (layer B.Cu) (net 3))
 (segment (start 120.65 119.7237) (end 125.73 119.7237) (width 1) (layer B.Cu) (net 3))
 (segment (start 124.3701 93.98) (end 125.9 93.98) (width 1) (layer F.Cu) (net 3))
 (segment (start 123.02 93.98) (end 124.3701 93.98) (width 1) (layer F.Cu) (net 3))
 (segment (start 125.9 93.98) (end 125.9 96.52) (width 1) (layer F.Cu) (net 3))
 (segment (start 125.9 96.52) (end 125.9 98.5463) (width 1) (layer F.Cu) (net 3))
 (segment (start 125.9 98.5463) (end 125.73 98.7163) (width 1) (layer F.Cu) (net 3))
 (segment (start 125.73 100.33) (end 125.73 98.7163) (width 1) (layer F.Cu) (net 3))
 (segment (start 142.2595 116.078) (end 141.3572 116.9803) (width 1) (layer F.Cu) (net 3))
 (segment (start 141.3572 116.9803) (end 132.2203 116.9803) (width 1) (layer F.Cu) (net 3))
 (segment (start 132.2203 116.9803) (end 130.81 115.57) (width 1) (layer F.Cu) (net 3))
 (segment (start 140.97 116.078) (end 142.2595 116.078) (width 1) (layer F.Cu) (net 3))
 (segment (start 140.97 122.682) (end 140.97 120.423) (width 1) (layer F.Cu) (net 3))
 (segment (start 140.97 120.423) (end 143.5489 117.8441) (width 1) (layer F.Cu) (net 3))
 (segment (start 143.5489 117.8441) (end 143.5489 116.078) (width 1) (layer F.Cu) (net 3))
 (segment (start 132.08 106.71) (end 128.3 110.49) (width 1) (layer F.Cu) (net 3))
 (segment (start 128.3 110.49) (end 125.73 110.49) (width 1) (layer F.Cu) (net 3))
 (via (at 150.0663 101.5302) (size 1) (drill 0.8) (layers F.Cu B.Cu) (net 3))
 (segment (start 152.32 97.79) (end 152.32 97.88) (width 0.25) (layer F.Cu) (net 4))
 (segment (start 152.32 97.88) (end 154.77 100.33) (width 0.25) (layer F.Cu) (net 4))
 (segment (start 161.29 102.87) (end 161.29 100.33) (width 0.25) (layer B.Cu) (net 5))
 (segment (start 161.29 100.33) (end 154.94 93.98) (width 0.25) (layer B.Cu) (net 5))
 (segment (start 161.29 105.41) (end 157.48 105.41) (width 0.25) (layer B.Cu) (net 6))
 (segment (start 157.48 105.41) (end 144.78 92.71) (width 0.25) (layer B.Cu) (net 6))
 (segment (start 144.78 92.71) (end 148.08 92.71) (width 0.25) (layer F.Cu) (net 6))
 (via (at 144.78 92.71) (size 0.6) (layers F.Cu B.Cu) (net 6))
 (segment (start 161.29 107.95) (end 154.94 107.95) (width 0.25) (layer B.Cu) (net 7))
 (segment (start 154.94 107.95) (end 142.24 95.25) (width 0.25) (layer B.Cu) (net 7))
 (segment (start 142.24 95.25) (end 142.78 94.71) (width 0.25) (layer F.Cu) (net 7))
 (segment (start 142.78 94.71) (end 148.08 94.71) (width 0.25) (layer F.Cu) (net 7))
 (via (at 142.24 95.25) (size 0.6) (layers F.Cu B.Cu) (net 7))
 (segment (start 148.24 102.87) (end 148.08 102.71) (width 0.25) (layer F.Cu) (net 10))
 (segment (start 156.21 106.51) (end 156.04 106.51) (width 0.25) (layer F.Cu) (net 10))
 (segment (start 156.04 106.51) (end 154.94 105.41) (width 0.25) (layer F.Cu) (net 10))
 (segment (start 154.94 105.41) (end 154.94 104.14) (width 0.25) (layer F.Cu) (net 10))
 (segment (start 154.94 104.14) (end 153.51 102.71) (width 0.25) (layer F.Cu) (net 10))
 (segment (start 153.51 102.71) (end 148.08 102.71) (width 0.25) (layer F.Cu) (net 10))
 (segment (start 148.08 102.71) (end 146.21 102.71) (width 0.25) (layer F.Cu) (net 10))
 (segment (start 146.21 102.71) (end 143.51 105.41) (width 0.25) (layer F.Cu) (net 10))
 (segment (start 143.51 105.41) (end 135.89 105.41) (width 0.25) (layer F.Cu) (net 10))
 (segment (start 135.89 105.41) (end 129.54 111.76) (width 0.25) (layer F.Cu) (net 10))
 (segment (start 129.54 111.76) (end 121.92 111.76) (width 0.25) (layer F.Cu) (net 10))
 (segment (start 121.92 111.76) (end 120.65 113.03) (width 0.25) (layer F.Cu) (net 10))
 (segment (start 132.08 102.71) (end 130.97 102.71) (width 0.25) (layer F.Cu) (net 11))
 (segment (start 130.97 102.71) (end 129.54 104.14) (width 0.25) (layer F.Cu) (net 11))
 (segment (start 129.54 104.14) (end 129.54 107.95) (width 0.25) (layer F.Cu) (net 11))
 (segment (start 129.54 107.95) (end 128.27 109.22) (width 0.25) (layer F.Cu) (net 11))
 (segment (start 128.27 109.22) (end 121.92 109.22) (width 0.25) (layer F.Cu) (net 11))
 (segment (start 121.92 109.22) (end 120.65 110.49) (width 0.25) (layer F.Cu) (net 11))
 (segment (start 132.08 100.71) (end 131.7 100.71) (width 0.25) (layer F.Cu) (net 12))
 (segment (start 131.7 100.71) (end 128.27 104.14) (width 0.25) (layer F.Cu) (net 12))
 (segment (start 128.27 104.14) (end 128.27 105.41) (width 0.25) (layer F.Cu) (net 12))
 (segment (start 128.27 105.41) (end 127 106.68) (width 0.25) (layer F.Cu) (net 12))
 (segment (start 127 106.68) (end 121.92 106.68) (width 0.25) (layer F.Cu) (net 12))
 (segment (start 121.92 106.68) (end 120.65 107.95) (width 0.25) (layer F.Cu) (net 12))
 (segment (start 132.08 98.71) (end 131.16 98.71) (width 0.25) (layer F.Cu) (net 13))
 (segment (start 131.16 98.71) (end 128.27 101.6) (width 0.25) (layer F.Cu) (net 13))
 (segment (start 128.27 101.6) (end 128.27 102.87) (width 0.25) (layer F.Cu) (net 13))
 (segment (start 128.27 102.87) (end 127 104.14) (width 0.25) (layer F.Cu) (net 13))
 (segment (start 127 104.14) (end 121.92 104.14) (width 0.25) (layer F.Cu) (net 13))
 (segment (start 121.92 104.14) (end 120.65 105.41) (width 0.25) (layer F.Cu) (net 13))
 (segment (start 132.08 104.71) (end 131.38 104.71) (width 0.25) (layer F.Cu) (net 14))
 (segment (start 118.11 99.06) (end 118.11 101.6) (width 0.25) (layer F.Cu) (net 14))
 (segment (start 118.11 101.6) (end 119.38 102.87) (width 0.25) (layer F.Cu) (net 14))
 (segment (start 119.38 102.87) (end 120.65 102.87) (width 0.25) (layer F.Cu) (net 14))
 (segment (start 135.89 104.14) (end 137.16 102.87) (width 0.25) (layer B.Cu) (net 14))
 (segment (start 137.16 102.87) (end 137.16 99.06) (width 0.25) (layer B.Cu) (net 14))
 (segment (start 137.16 99.06) (end 135.89 97.79) (width 0.25) (layer B.Cu) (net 14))
 (segment (start 135.89 97.79) (end 119.38 97.79) (width 0.25) (layer B.Cu) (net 14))
 (segment (start 119.38 97.79) (end 118.11 99.06) (width 0.25) (layer B.Cu) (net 14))
 (segment (start 132.08 104.71) (end 135.32 104.71) (width 0.25) (layer F.Cu) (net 14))
 (segment (start 135.32 104.71) (end 135.89 104.14) (width 0.25) (layer F.Cu) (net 14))
 (via (at 118.11 99.06) (size 0.6) (layers F.Cu B.Cu) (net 14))
 (via (at 135.89 104.14) (size 0.6) (layers F.Cu B.Cu) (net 14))
 (segment (start 120.82 93.98) (end 120.65 94.15) (width 0.25) (layer F.Cu) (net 15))
 (segment (start 120.65 94.15) (end 120.65 100.33) (width 0.25) (layer F.Cu) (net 15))
 (segment (start 123.19 96.52) (end 120.82 94.15) (width 0.25) (layer F.Cu) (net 15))
 (segment (start 120.82 94.15) (end 120.82 93.98) (width 0.25) (layer F.Cu) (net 15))
 (segment (start 134.62 96.52) (end 123.19 96.52) (width 0.25) (layer B.Cu) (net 15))
 (segment (start 132.08 94.71) (end 132.81 94.71) (width 0.25) (layer F.Cu) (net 15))
 (segment (start 132.81 94.71) (end 134.62 96.52) (width 0.25) (layer F.Cu) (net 15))
 (via (at 123.19 96.52) (size 0.6) (layers F.Cu B.Cu) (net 15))
 (via (at 134.62 96.52) (size 0.6) (layers F.Cu B.Cu) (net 15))
 (segment (start 128.1 96.52) (end 131.89 96.52) (width 0.25) (layer F.Cu) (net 16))
 (segment (start 131.89 96.52) (end 132.08 96.71) (width 0.25) (layer F.Cu) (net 16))
 (segment (start 129 90.505) (end 129 84.755) (width 0.25) (layer F.Cu) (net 17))
 (segment (start 128.1 93.98) (end 128.1 91.405) (width 0.25) (layer F.Cu) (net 17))
 (segment (start 128.1 91.405) (end 129 90.505) (width 0.25) (layer F.Cu) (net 17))
 (segment (start 161.29 93.98) (end 161.29 92.71) (width 0.25) (layer B.Cu) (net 17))
 (segment (start 161.29 92.71) (end 156.21 87.63) (width 0.25) (layer B.Cu) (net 17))
 (segment (start 156.21 87.63) (end 151.13 87.63) (width 0.25) (layer B.Cu) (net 17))
 (segment (start 151.13 87.63) (end 147.32 91.44) (width 0.25) (layer B.Cu) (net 17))
 (segment (start 147.32 91.44) (end 138.43 91.44) (width 0.25) (layer B.Cu) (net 17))
 (segment (start 138.43 91.44) (end 137.16 92.71) (width 0.25) (layer F.Cu) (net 17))
 (segment (start 137.16 92.71) (end 132.08 92.71) (width 0.25) (layer F.Cu) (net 17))
 (segment (start 132.08 92.71) (end 129.37 92.71) (width 0.25) (layer F.Cu) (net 17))
 (segment (start 129.37 92.71) (end 128.1 93.98) (width 0.25) (layer F.Cu) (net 17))
 (via (at 138.43 91.44) (size 0.6) (layers F.Cu B.Cu) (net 17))
 (segment (start 151.67 90.505) (end 151.67 84.755) (width 0.25) (layer F.Cu) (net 18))
 (segment (start 152.57 100.33) (end 152.4 100.33) (width 0.25) (layer F.Cu) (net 18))
 (segment (start 152.4 100.33) (end 149.86 97.79) (width 0.25) (layer F.Cu) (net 18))
 (segment (start 149.86 97.79) (end 149.86 92.315) (width 0.25) (layer F.Cu) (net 18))
 (segment (start 149.86 92.315) (end 151.67 90.505) (width 0.25) (layer F.Cu) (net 18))
 (segment (start 152.57 100.33) (end 148.46 100.33) (width 0.25) (layer F.Cu) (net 18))
 (segment (start 148.46 100.33) (end 148.08 100.71) (width 0.25) (layer F.Cu) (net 18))
 (segment (start 152.4 93.98) (end 152.4 91.235) (width 0.25) (layer F.Cu) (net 18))
 (segment (start 152.4 91.235) (end 151.67 90.505) (width 0.25) (layer F.Cu) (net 18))
 (segment (start 148.78 105.41) (end 148.08 104.71) (width 0.25) (layer F.Cu) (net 19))
 (segment (start 152.4 104.31) (end 148.48 104.31) (width 0.25) (layer F.Cu) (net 19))
 (segment (start 148.48 104.31) (end 148.08 104.71) (width 0.25) (layer F.Cu) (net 19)))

